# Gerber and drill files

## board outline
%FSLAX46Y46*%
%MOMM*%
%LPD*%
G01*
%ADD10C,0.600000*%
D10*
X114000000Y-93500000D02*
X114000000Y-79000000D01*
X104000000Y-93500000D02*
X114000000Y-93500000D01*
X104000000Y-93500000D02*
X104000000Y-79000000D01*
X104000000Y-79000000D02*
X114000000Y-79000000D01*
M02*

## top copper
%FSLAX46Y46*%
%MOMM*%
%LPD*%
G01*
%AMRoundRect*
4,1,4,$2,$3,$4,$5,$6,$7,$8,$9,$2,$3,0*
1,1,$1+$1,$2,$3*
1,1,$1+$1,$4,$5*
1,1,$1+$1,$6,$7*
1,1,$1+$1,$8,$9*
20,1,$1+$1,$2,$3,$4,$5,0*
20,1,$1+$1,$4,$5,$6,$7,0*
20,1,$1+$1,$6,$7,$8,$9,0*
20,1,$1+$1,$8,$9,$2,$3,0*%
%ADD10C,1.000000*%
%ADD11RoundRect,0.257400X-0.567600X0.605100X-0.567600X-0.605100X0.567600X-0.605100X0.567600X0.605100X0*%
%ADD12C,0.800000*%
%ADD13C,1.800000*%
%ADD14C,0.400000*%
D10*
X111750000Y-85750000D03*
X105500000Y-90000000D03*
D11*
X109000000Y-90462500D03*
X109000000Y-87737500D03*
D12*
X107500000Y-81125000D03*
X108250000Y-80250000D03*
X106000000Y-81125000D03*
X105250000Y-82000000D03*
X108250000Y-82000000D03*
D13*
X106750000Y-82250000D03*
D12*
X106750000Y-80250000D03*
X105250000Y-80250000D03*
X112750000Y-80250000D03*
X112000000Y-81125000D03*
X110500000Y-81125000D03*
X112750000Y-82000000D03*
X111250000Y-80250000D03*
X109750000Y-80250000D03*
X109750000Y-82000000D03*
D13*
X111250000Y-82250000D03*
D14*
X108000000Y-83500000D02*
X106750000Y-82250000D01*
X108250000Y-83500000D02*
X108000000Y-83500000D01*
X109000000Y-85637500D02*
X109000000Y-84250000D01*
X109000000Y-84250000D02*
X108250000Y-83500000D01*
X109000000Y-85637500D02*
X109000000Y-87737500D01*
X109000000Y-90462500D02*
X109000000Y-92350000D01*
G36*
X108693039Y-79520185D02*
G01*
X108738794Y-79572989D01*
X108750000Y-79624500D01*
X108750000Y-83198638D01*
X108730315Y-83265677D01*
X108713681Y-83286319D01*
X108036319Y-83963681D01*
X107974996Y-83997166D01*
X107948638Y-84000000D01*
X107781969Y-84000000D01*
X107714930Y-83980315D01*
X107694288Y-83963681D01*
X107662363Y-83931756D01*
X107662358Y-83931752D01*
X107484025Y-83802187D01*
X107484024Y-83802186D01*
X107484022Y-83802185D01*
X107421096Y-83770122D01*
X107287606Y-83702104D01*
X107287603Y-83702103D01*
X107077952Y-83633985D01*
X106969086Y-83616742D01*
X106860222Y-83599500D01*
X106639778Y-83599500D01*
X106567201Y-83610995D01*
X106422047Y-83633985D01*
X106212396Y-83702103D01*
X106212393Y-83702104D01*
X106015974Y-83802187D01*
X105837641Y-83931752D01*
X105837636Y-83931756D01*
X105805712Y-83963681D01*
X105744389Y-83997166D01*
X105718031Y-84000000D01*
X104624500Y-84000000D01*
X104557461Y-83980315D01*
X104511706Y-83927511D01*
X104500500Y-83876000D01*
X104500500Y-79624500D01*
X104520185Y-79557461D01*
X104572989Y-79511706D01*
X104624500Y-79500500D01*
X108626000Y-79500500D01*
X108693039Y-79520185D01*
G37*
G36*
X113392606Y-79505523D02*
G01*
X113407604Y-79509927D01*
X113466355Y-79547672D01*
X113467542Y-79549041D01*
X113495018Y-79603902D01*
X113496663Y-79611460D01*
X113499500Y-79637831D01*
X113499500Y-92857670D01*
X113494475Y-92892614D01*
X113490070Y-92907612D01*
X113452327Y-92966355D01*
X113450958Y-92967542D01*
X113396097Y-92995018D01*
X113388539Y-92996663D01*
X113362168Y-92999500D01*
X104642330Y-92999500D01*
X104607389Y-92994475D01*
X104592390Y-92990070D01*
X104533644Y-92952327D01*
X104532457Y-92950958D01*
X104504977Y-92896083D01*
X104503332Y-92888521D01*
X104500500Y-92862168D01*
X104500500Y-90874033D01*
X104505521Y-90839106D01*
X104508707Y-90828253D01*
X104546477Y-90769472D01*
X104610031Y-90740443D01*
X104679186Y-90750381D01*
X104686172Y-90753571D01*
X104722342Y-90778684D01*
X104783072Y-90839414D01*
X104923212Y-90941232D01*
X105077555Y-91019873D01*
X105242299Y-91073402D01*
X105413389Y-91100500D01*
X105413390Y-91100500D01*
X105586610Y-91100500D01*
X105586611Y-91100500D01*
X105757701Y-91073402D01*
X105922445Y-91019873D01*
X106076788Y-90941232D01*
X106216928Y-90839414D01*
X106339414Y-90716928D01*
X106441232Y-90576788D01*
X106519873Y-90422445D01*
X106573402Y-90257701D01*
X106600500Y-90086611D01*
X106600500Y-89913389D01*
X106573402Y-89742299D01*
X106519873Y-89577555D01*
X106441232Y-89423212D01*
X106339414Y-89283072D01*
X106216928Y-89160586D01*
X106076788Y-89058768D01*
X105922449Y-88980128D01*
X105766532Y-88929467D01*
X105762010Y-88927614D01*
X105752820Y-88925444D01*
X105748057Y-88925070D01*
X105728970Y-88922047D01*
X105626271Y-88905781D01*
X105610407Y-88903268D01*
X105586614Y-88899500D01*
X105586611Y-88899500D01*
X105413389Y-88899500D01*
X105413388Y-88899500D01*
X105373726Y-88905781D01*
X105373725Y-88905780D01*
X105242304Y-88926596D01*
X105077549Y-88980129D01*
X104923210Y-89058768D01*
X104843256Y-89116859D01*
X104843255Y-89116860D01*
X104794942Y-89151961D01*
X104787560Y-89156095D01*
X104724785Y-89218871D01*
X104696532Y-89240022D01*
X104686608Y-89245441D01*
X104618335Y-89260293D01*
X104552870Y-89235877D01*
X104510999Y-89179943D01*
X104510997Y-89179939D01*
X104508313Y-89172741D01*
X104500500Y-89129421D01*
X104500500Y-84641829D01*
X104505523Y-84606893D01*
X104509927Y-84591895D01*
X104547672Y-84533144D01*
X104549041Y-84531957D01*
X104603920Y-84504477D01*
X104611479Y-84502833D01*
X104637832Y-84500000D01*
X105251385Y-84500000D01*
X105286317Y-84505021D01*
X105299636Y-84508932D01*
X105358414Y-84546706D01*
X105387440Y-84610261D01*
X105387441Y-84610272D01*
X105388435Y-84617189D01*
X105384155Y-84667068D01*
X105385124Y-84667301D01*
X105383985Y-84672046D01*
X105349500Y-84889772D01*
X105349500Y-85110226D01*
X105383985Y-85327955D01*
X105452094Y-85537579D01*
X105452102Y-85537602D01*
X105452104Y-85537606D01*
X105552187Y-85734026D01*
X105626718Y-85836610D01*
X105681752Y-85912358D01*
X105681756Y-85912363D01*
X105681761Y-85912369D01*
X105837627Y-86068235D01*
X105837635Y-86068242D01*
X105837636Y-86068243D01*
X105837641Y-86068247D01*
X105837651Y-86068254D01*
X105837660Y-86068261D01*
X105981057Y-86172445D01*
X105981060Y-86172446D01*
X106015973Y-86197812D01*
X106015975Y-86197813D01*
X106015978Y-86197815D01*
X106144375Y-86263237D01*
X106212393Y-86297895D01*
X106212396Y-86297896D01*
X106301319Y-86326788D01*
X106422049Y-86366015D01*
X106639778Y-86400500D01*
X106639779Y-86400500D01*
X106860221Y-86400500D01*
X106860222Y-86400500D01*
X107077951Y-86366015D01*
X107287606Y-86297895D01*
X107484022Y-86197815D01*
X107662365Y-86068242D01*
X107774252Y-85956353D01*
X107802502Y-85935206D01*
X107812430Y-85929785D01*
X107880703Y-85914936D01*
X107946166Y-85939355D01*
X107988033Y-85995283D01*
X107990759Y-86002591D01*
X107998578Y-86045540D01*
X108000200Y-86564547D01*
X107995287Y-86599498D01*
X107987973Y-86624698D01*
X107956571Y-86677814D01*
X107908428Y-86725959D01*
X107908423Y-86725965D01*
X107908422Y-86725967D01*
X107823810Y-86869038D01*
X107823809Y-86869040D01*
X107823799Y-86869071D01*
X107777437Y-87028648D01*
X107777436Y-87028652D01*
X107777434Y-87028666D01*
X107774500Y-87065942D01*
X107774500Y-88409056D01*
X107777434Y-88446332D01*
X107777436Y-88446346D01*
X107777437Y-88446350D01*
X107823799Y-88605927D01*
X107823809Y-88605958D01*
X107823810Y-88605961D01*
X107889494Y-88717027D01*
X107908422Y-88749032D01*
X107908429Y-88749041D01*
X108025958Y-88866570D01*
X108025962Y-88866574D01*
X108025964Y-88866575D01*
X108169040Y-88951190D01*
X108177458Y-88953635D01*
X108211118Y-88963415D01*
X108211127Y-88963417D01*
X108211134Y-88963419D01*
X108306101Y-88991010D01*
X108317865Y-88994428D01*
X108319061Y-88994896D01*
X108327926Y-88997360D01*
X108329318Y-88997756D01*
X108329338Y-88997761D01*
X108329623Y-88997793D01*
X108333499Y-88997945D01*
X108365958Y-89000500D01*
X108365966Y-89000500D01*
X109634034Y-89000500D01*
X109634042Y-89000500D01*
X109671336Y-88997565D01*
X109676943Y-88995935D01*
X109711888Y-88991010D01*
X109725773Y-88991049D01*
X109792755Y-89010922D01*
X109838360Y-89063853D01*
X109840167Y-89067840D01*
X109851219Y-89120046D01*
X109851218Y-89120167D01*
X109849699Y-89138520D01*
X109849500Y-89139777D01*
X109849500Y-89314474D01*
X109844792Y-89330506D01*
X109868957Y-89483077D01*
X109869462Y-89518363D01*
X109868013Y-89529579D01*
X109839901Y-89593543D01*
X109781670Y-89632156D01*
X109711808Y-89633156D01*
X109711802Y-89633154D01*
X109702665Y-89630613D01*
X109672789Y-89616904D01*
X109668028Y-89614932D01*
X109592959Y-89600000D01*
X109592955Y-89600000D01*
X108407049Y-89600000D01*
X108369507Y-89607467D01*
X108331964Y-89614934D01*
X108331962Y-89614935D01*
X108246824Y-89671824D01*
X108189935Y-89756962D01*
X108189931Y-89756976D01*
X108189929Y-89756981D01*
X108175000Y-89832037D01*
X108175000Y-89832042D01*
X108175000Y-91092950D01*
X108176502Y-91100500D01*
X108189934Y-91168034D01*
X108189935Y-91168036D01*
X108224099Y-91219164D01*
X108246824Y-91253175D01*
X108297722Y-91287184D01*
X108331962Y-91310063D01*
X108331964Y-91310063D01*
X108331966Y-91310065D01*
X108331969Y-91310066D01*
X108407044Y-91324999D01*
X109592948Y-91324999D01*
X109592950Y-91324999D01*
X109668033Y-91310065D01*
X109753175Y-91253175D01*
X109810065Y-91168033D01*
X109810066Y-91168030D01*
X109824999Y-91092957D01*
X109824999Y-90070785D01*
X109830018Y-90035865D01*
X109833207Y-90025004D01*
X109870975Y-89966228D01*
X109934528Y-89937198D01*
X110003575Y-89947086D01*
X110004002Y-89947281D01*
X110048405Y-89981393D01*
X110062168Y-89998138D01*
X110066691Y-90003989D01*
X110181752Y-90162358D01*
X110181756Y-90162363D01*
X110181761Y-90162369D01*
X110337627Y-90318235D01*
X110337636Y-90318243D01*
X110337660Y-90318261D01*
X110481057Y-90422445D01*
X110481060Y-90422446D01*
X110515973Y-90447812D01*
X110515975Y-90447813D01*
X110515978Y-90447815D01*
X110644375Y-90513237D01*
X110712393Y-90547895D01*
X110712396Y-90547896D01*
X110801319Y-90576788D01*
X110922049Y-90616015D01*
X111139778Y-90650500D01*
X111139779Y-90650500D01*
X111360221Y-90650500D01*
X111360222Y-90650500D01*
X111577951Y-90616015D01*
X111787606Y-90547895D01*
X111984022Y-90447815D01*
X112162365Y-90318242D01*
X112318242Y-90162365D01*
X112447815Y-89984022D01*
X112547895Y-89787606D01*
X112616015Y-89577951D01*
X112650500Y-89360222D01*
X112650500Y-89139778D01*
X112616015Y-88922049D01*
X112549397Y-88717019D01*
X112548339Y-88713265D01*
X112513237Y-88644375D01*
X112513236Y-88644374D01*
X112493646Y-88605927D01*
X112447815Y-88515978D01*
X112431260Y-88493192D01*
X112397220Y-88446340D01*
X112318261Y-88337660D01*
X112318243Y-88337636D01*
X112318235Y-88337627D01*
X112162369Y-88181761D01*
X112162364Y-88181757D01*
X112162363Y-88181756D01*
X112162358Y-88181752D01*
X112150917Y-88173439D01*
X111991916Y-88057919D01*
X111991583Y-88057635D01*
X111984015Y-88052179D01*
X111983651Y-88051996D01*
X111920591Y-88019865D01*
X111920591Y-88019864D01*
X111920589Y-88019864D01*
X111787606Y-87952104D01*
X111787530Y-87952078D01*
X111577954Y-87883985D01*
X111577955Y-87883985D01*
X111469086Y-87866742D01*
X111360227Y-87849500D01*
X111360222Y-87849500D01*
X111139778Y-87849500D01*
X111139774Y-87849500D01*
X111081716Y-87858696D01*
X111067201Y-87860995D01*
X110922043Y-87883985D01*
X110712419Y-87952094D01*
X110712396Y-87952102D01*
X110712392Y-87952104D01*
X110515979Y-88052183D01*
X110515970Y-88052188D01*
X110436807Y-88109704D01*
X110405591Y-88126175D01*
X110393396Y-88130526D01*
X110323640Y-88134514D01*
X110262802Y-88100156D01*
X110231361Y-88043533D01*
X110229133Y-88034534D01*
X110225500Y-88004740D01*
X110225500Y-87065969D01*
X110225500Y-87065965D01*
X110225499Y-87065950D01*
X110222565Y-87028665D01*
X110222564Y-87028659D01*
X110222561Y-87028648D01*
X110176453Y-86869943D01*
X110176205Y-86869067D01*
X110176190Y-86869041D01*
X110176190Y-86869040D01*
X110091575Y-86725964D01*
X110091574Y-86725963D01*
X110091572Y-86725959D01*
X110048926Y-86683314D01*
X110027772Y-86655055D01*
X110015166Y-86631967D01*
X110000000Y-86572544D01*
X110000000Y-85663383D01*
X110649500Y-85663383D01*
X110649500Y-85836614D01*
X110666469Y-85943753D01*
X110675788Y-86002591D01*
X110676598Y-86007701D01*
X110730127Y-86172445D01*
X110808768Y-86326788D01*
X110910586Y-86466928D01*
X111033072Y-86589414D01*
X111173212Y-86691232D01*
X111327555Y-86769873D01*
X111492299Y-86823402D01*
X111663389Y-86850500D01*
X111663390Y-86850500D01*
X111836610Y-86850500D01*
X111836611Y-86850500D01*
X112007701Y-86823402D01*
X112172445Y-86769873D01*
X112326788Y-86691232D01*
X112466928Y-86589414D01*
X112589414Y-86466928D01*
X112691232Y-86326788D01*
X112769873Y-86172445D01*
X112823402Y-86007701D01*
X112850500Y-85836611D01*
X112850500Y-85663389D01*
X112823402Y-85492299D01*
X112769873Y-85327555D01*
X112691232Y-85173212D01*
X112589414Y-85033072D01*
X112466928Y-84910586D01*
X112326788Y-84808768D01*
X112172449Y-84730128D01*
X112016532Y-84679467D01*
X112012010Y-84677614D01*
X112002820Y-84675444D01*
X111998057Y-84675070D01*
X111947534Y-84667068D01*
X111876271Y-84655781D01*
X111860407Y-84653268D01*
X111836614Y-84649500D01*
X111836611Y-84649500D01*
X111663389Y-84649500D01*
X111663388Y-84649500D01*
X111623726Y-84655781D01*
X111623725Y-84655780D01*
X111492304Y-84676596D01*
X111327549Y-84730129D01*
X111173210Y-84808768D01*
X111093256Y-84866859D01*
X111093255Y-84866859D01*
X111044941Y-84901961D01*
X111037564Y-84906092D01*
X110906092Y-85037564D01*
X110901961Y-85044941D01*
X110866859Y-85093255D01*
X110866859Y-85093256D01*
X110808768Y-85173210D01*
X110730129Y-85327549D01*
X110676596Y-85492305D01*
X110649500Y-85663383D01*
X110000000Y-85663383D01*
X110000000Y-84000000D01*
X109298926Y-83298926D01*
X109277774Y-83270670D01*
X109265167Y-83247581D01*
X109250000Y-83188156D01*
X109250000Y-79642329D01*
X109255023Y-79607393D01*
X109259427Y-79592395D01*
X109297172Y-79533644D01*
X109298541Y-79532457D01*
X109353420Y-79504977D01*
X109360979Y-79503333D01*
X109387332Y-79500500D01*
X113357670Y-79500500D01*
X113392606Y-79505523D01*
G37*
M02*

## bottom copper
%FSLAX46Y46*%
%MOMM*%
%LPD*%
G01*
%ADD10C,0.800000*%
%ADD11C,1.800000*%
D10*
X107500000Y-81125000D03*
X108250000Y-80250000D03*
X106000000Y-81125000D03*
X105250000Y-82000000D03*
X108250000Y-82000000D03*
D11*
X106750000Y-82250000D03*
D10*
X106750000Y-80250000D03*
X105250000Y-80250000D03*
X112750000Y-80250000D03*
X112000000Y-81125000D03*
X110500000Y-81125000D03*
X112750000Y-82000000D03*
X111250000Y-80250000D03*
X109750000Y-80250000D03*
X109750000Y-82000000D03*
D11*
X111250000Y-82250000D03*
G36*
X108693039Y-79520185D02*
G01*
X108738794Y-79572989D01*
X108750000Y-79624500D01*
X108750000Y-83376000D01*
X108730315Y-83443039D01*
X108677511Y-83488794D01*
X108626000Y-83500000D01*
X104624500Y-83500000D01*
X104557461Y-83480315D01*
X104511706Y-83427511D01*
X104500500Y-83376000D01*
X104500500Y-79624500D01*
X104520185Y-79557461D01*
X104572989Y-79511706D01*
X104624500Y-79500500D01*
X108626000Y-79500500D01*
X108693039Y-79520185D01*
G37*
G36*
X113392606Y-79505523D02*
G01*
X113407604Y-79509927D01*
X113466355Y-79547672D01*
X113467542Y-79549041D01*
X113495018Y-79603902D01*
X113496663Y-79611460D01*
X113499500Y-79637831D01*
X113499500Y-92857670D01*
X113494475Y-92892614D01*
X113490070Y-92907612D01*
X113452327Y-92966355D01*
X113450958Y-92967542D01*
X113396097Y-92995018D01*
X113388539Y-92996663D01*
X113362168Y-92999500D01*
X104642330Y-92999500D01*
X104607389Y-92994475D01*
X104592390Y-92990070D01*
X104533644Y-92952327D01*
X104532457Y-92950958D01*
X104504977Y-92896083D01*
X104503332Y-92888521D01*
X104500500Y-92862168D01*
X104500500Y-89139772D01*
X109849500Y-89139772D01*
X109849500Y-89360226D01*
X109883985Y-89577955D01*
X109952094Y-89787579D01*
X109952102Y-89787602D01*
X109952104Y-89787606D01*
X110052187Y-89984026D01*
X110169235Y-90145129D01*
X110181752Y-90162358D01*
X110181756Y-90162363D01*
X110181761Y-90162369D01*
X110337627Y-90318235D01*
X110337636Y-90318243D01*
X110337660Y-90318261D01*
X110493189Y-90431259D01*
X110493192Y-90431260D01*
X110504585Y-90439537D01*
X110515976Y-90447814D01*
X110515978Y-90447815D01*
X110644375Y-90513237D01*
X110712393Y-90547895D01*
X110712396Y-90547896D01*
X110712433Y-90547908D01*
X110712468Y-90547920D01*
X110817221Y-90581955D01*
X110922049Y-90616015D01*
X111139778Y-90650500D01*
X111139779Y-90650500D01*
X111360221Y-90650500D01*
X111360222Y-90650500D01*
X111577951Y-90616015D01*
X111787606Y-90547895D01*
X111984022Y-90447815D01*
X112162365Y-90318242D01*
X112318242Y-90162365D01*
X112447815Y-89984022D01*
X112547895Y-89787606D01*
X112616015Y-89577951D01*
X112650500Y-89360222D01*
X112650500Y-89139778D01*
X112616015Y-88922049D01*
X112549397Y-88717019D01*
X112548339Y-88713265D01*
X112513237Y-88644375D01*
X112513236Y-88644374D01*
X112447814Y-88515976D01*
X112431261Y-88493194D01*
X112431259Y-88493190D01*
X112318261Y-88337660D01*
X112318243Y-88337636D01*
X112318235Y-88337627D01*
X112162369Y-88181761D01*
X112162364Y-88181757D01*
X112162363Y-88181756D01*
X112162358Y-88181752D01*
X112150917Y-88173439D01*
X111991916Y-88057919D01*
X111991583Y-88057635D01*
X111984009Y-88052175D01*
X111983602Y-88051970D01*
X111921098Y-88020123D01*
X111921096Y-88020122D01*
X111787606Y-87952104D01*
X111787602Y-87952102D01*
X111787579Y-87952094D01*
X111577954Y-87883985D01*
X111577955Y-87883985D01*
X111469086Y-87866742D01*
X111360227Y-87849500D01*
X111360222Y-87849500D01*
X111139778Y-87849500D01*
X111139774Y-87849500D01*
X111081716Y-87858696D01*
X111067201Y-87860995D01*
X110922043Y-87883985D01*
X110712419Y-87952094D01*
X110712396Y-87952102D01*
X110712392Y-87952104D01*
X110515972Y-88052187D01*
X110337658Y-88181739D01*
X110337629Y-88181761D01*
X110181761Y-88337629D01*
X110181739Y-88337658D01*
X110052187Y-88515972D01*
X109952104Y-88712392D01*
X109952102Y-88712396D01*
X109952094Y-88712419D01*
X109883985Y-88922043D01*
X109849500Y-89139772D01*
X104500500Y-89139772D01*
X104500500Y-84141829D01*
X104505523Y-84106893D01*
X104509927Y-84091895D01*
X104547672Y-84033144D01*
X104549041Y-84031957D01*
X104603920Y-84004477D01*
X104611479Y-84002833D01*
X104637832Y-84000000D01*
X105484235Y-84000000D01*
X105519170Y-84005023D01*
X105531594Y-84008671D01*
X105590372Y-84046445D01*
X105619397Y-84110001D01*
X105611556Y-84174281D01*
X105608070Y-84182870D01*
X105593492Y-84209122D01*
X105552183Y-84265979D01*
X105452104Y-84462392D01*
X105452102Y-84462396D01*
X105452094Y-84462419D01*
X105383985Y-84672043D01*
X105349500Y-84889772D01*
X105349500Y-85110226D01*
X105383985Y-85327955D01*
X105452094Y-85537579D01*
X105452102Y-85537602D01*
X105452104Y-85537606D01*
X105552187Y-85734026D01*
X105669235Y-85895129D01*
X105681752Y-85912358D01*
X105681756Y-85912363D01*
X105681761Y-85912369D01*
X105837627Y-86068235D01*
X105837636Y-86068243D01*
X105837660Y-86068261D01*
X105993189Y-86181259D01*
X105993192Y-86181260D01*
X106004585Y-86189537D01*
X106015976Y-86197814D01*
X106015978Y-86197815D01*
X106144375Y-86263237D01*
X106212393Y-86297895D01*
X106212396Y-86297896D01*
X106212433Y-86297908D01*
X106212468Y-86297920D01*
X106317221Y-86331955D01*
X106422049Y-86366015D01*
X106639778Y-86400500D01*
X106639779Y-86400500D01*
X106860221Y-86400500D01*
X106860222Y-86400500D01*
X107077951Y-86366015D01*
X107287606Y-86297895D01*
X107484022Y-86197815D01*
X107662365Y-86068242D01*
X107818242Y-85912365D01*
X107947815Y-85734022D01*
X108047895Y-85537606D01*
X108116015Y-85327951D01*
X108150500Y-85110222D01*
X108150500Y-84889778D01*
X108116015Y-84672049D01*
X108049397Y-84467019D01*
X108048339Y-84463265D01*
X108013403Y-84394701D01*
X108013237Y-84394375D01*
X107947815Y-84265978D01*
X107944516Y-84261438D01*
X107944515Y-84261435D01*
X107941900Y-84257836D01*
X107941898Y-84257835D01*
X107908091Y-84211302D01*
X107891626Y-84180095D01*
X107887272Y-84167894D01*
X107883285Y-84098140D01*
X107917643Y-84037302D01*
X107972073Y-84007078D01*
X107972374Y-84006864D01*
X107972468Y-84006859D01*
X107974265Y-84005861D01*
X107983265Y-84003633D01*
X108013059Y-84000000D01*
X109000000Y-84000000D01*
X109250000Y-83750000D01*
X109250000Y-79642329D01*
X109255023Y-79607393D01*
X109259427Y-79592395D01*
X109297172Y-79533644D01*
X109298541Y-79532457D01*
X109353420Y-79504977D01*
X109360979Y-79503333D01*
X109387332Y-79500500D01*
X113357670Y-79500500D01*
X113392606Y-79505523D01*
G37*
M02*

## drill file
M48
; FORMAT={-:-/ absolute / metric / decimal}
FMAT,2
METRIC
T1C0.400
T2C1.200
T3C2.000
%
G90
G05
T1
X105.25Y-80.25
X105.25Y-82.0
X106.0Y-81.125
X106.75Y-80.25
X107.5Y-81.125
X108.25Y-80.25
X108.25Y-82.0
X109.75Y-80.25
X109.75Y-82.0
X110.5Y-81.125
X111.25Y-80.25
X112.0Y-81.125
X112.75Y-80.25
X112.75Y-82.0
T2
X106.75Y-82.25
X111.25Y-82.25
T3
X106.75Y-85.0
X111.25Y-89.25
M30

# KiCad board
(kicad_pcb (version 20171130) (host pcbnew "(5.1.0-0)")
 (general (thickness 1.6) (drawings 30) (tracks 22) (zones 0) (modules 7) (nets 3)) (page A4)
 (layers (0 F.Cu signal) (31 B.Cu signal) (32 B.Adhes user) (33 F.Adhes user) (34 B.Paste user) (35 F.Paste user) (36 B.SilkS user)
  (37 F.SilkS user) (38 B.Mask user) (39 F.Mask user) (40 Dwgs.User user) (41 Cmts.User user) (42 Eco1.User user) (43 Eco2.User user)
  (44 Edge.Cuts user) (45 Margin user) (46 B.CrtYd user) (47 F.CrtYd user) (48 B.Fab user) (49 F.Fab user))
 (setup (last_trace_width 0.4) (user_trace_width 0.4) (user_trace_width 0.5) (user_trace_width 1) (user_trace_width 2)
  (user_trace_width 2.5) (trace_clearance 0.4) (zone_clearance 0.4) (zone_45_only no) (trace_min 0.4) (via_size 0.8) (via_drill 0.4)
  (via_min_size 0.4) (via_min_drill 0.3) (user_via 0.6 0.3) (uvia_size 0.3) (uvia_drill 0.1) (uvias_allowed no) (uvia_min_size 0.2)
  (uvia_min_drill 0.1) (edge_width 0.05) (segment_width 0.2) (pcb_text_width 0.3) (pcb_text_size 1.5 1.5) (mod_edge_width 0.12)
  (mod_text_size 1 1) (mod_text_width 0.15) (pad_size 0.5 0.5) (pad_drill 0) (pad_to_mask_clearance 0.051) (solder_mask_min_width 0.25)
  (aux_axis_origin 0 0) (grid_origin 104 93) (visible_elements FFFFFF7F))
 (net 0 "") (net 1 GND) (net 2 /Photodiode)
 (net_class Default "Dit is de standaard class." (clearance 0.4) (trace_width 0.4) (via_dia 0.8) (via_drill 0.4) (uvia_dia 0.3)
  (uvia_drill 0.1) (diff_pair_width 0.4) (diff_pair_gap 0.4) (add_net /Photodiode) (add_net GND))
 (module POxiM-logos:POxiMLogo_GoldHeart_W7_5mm (layer F.Cu) (at 109 92.3)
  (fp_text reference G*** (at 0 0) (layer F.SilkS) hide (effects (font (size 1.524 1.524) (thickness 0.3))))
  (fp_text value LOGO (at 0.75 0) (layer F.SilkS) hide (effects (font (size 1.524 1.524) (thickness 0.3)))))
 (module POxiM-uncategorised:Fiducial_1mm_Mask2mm (layer F.Cu) (at 111.75 85.75)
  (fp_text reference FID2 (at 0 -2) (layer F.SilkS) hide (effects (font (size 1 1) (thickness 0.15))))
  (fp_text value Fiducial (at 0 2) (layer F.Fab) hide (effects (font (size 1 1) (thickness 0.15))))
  (pad "" smd circle (at 0 0) (size 1 1) (layers F.Cu F.Mask) (solder_mask_margin 0.5) (clearance 0.6)))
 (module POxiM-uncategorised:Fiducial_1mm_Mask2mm (layer F.Cu) (at 105.5 90)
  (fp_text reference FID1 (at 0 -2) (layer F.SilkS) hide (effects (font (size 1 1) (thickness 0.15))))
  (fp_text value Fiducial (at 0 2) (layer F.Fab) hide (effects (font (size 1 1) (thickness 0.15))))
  (pad "" smd circle (at 0 0) (size 1 1) (layers F.Cu F.Mask) (solder_mask_margin 0.5) (clearance 0.6)))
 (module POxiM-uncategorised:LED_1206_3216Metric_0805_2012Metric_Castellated (layer F.Cu) (at 109 89.1 270) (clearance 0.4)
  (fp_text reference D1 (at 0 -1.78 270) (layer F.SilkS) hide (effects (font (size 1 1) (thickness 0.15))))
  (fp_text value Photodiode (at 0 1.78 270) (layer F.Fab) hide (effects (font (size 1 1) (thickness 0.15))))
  (pad 2 smd roundrect (at 1.3625 0 270) (size 1.725 1.65) (layers F.Cu F.Paste F.Mask) (roundrect_rratio 0.156) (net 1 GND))
  (pad 1 smd roundrect (at -1.3625 0 270) (size 1.725 1.65) (layers F.Cu F.Paste F.Mask) (roundrect_rratio 0.156) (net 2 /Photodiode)))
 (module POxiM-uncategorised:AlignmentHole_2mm (layer F.Cu) (at 106.75 85) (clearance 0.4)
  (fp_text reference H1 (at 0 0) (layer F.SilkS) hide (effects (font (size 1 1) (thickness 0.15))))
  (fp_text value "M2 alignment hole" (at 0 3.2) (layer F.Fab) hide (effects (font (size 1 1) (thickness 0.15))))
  (pad "" np_thru_hole circle (at 0 0) (size 2 2) (drill 2) (layers *.Cu *.Mask)))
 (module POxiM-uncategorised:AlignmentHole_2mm (layer F.Cu) (at 111.25 89.25) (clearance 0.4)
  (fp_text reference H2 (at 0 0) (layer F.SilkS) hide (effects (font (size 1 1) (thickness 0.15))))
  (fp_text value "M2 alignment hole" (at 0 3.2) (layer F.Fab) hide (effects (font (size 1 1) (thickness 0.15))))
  (pad "" np_thru_hole circle (at 0 0) (size 2 2) (drill 2) (layers *.Cu *.Mask)))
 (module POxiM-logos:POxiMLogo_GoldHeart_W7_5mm (layer B.Cu) (at 109 87.25)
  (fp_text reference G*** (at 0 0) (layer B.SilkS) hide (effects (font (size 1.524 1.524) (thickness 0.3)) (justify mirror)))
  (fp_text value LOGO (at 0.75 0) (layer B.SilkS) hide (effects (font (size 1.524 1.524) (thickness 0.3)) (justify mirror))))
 (gr_line (start 114 93.5) (end 114 79) (layer Edge.Cuts) (width 0.6))
 (gr_line (start 104 93.5) (end 114 93.5) (layer Edge.Cuts) (width 0.6))
 (gr_line (start 104 93.5) (end 104 79) (layer Edge.Cuts) (width 0.6))
 (gr_line (start 104 79) (end 114 79) (layer Edge.Cuts) (width 0.6))
 (via (at 107.5 81.125) (size 0.8) (drill 0.4) (layers F.Cu B.Cu) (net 2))
 (via (at 108.25 80.25) (size 0.8) (drill 0.4) (layers F.Cu B.Cu) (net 2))
 (via (at 106 81.125) (size 0.8) (drill 0.4) (layers F.Cu B.Cu) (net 2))
 (via (at 105.25 82) (size 0.8) (drill 0.4) (layers F.Cu B.Cu) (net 2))
 (via (at 108.25 82) (size 0.8) (drill 0.4) (layers F.Cu B.Cu) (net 2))
 (via (at 106.75 82.25) (size 1.8) (drill 1.2) (layers F.Cu B.Cu) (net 2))
 (via (at 106.75 80.25) (size 0.8) (drill 0.4) (layers F.Cu B.Cu) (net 2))
 (via (at 105.25 80.25) (size 0.8) (drill 0.4) (layers F.Cu B.Cu) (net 2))
 (segment (start 108 83.5) (end 106.75 82.25) (width 0.4) (layer F.Cu) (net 2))
 (segment (start 108.25 83.5) (end 108 83.5) (width 0.4) (layer F.Cu) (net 2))
 (segment (start 109 85.6375) (end 109 84.25) (width 0.4) (layer F.Cu) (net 2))
 (segment (start 109 84.25) (end 108.25 83.5) (width 0.4) (layer F.Cu) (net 2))
 (segment (start 109 85.6375) (end 109 87.7375) (width 0.4) (layer F.Cu) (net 2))
 (via (at 112.75 80.25) (size 0.8) (drill 0.4) (layers F.Cu B.Cu) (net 1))
 (via (at 112 81.125) (size 0.8) (drill 0.4) (layers F.Cu B.Cu) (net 1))
 (via (at 110.5 81.125) (size 0.8) (drill 0.4) (layers F.Cu B.Cu) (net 1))
 (via (at 112.75 82) (size 0.8) (drill 0.4) (layers F.Cu B.Cu) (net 1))
 (via (at 111.25 80.25) (size 0.8) (drill 0.4) (layers F.Cu B.Cu) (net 1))
 (via (at 109.75 80.25) (size 0.8) (drill 0.4) (layers F.Cu B.Cu) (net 1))
 (via (at 109.75 82) (size 0.8) (drill 0.4) (layers F.Cu B.Cu) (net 1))
 (via (at 111.25 82.25) (size 1.8) (drill 1.2) (layers F.Cu B.Cu) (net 1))
 (segment (start 109 90.4625) (end 109 92.35) (width 0.4) (layer F.Cu) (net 1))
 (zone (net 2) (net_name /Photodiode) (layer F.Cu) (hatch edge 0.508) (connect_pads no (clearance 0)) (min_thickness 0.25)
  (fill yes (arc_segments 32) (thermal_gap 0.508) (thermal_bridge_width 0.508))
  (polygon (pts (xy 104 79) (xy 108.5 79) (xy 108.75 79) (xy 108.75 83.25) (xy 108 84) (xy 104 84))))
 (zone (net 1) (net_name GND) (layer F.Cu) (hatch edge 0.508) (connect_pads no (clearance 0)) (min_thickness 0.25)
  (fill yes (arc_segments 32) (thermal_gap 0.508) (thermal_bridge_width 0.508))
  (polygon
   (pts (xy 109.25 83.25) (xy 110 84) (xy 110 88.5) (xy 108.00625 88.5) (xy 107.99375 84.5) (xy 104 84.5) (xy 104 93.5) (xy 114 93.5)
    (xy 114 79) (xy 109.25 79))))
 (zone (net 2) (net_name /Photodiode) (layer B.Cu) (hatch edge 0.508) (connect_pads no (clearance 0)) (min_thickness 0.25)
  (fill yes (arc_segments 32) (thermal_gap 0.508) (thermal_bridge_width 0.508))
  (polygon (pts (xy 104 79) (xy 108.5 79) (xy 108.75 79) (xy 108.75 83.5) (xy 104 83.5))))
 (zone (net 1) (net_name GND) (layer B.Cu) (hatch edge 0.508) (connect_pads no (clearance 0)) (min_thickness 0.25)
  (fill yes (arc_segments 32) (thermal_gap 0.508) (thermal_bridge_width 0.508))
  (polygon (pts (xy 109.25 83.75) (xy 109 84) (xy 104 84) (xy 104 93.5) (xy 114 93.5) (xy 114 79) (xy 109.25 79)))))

